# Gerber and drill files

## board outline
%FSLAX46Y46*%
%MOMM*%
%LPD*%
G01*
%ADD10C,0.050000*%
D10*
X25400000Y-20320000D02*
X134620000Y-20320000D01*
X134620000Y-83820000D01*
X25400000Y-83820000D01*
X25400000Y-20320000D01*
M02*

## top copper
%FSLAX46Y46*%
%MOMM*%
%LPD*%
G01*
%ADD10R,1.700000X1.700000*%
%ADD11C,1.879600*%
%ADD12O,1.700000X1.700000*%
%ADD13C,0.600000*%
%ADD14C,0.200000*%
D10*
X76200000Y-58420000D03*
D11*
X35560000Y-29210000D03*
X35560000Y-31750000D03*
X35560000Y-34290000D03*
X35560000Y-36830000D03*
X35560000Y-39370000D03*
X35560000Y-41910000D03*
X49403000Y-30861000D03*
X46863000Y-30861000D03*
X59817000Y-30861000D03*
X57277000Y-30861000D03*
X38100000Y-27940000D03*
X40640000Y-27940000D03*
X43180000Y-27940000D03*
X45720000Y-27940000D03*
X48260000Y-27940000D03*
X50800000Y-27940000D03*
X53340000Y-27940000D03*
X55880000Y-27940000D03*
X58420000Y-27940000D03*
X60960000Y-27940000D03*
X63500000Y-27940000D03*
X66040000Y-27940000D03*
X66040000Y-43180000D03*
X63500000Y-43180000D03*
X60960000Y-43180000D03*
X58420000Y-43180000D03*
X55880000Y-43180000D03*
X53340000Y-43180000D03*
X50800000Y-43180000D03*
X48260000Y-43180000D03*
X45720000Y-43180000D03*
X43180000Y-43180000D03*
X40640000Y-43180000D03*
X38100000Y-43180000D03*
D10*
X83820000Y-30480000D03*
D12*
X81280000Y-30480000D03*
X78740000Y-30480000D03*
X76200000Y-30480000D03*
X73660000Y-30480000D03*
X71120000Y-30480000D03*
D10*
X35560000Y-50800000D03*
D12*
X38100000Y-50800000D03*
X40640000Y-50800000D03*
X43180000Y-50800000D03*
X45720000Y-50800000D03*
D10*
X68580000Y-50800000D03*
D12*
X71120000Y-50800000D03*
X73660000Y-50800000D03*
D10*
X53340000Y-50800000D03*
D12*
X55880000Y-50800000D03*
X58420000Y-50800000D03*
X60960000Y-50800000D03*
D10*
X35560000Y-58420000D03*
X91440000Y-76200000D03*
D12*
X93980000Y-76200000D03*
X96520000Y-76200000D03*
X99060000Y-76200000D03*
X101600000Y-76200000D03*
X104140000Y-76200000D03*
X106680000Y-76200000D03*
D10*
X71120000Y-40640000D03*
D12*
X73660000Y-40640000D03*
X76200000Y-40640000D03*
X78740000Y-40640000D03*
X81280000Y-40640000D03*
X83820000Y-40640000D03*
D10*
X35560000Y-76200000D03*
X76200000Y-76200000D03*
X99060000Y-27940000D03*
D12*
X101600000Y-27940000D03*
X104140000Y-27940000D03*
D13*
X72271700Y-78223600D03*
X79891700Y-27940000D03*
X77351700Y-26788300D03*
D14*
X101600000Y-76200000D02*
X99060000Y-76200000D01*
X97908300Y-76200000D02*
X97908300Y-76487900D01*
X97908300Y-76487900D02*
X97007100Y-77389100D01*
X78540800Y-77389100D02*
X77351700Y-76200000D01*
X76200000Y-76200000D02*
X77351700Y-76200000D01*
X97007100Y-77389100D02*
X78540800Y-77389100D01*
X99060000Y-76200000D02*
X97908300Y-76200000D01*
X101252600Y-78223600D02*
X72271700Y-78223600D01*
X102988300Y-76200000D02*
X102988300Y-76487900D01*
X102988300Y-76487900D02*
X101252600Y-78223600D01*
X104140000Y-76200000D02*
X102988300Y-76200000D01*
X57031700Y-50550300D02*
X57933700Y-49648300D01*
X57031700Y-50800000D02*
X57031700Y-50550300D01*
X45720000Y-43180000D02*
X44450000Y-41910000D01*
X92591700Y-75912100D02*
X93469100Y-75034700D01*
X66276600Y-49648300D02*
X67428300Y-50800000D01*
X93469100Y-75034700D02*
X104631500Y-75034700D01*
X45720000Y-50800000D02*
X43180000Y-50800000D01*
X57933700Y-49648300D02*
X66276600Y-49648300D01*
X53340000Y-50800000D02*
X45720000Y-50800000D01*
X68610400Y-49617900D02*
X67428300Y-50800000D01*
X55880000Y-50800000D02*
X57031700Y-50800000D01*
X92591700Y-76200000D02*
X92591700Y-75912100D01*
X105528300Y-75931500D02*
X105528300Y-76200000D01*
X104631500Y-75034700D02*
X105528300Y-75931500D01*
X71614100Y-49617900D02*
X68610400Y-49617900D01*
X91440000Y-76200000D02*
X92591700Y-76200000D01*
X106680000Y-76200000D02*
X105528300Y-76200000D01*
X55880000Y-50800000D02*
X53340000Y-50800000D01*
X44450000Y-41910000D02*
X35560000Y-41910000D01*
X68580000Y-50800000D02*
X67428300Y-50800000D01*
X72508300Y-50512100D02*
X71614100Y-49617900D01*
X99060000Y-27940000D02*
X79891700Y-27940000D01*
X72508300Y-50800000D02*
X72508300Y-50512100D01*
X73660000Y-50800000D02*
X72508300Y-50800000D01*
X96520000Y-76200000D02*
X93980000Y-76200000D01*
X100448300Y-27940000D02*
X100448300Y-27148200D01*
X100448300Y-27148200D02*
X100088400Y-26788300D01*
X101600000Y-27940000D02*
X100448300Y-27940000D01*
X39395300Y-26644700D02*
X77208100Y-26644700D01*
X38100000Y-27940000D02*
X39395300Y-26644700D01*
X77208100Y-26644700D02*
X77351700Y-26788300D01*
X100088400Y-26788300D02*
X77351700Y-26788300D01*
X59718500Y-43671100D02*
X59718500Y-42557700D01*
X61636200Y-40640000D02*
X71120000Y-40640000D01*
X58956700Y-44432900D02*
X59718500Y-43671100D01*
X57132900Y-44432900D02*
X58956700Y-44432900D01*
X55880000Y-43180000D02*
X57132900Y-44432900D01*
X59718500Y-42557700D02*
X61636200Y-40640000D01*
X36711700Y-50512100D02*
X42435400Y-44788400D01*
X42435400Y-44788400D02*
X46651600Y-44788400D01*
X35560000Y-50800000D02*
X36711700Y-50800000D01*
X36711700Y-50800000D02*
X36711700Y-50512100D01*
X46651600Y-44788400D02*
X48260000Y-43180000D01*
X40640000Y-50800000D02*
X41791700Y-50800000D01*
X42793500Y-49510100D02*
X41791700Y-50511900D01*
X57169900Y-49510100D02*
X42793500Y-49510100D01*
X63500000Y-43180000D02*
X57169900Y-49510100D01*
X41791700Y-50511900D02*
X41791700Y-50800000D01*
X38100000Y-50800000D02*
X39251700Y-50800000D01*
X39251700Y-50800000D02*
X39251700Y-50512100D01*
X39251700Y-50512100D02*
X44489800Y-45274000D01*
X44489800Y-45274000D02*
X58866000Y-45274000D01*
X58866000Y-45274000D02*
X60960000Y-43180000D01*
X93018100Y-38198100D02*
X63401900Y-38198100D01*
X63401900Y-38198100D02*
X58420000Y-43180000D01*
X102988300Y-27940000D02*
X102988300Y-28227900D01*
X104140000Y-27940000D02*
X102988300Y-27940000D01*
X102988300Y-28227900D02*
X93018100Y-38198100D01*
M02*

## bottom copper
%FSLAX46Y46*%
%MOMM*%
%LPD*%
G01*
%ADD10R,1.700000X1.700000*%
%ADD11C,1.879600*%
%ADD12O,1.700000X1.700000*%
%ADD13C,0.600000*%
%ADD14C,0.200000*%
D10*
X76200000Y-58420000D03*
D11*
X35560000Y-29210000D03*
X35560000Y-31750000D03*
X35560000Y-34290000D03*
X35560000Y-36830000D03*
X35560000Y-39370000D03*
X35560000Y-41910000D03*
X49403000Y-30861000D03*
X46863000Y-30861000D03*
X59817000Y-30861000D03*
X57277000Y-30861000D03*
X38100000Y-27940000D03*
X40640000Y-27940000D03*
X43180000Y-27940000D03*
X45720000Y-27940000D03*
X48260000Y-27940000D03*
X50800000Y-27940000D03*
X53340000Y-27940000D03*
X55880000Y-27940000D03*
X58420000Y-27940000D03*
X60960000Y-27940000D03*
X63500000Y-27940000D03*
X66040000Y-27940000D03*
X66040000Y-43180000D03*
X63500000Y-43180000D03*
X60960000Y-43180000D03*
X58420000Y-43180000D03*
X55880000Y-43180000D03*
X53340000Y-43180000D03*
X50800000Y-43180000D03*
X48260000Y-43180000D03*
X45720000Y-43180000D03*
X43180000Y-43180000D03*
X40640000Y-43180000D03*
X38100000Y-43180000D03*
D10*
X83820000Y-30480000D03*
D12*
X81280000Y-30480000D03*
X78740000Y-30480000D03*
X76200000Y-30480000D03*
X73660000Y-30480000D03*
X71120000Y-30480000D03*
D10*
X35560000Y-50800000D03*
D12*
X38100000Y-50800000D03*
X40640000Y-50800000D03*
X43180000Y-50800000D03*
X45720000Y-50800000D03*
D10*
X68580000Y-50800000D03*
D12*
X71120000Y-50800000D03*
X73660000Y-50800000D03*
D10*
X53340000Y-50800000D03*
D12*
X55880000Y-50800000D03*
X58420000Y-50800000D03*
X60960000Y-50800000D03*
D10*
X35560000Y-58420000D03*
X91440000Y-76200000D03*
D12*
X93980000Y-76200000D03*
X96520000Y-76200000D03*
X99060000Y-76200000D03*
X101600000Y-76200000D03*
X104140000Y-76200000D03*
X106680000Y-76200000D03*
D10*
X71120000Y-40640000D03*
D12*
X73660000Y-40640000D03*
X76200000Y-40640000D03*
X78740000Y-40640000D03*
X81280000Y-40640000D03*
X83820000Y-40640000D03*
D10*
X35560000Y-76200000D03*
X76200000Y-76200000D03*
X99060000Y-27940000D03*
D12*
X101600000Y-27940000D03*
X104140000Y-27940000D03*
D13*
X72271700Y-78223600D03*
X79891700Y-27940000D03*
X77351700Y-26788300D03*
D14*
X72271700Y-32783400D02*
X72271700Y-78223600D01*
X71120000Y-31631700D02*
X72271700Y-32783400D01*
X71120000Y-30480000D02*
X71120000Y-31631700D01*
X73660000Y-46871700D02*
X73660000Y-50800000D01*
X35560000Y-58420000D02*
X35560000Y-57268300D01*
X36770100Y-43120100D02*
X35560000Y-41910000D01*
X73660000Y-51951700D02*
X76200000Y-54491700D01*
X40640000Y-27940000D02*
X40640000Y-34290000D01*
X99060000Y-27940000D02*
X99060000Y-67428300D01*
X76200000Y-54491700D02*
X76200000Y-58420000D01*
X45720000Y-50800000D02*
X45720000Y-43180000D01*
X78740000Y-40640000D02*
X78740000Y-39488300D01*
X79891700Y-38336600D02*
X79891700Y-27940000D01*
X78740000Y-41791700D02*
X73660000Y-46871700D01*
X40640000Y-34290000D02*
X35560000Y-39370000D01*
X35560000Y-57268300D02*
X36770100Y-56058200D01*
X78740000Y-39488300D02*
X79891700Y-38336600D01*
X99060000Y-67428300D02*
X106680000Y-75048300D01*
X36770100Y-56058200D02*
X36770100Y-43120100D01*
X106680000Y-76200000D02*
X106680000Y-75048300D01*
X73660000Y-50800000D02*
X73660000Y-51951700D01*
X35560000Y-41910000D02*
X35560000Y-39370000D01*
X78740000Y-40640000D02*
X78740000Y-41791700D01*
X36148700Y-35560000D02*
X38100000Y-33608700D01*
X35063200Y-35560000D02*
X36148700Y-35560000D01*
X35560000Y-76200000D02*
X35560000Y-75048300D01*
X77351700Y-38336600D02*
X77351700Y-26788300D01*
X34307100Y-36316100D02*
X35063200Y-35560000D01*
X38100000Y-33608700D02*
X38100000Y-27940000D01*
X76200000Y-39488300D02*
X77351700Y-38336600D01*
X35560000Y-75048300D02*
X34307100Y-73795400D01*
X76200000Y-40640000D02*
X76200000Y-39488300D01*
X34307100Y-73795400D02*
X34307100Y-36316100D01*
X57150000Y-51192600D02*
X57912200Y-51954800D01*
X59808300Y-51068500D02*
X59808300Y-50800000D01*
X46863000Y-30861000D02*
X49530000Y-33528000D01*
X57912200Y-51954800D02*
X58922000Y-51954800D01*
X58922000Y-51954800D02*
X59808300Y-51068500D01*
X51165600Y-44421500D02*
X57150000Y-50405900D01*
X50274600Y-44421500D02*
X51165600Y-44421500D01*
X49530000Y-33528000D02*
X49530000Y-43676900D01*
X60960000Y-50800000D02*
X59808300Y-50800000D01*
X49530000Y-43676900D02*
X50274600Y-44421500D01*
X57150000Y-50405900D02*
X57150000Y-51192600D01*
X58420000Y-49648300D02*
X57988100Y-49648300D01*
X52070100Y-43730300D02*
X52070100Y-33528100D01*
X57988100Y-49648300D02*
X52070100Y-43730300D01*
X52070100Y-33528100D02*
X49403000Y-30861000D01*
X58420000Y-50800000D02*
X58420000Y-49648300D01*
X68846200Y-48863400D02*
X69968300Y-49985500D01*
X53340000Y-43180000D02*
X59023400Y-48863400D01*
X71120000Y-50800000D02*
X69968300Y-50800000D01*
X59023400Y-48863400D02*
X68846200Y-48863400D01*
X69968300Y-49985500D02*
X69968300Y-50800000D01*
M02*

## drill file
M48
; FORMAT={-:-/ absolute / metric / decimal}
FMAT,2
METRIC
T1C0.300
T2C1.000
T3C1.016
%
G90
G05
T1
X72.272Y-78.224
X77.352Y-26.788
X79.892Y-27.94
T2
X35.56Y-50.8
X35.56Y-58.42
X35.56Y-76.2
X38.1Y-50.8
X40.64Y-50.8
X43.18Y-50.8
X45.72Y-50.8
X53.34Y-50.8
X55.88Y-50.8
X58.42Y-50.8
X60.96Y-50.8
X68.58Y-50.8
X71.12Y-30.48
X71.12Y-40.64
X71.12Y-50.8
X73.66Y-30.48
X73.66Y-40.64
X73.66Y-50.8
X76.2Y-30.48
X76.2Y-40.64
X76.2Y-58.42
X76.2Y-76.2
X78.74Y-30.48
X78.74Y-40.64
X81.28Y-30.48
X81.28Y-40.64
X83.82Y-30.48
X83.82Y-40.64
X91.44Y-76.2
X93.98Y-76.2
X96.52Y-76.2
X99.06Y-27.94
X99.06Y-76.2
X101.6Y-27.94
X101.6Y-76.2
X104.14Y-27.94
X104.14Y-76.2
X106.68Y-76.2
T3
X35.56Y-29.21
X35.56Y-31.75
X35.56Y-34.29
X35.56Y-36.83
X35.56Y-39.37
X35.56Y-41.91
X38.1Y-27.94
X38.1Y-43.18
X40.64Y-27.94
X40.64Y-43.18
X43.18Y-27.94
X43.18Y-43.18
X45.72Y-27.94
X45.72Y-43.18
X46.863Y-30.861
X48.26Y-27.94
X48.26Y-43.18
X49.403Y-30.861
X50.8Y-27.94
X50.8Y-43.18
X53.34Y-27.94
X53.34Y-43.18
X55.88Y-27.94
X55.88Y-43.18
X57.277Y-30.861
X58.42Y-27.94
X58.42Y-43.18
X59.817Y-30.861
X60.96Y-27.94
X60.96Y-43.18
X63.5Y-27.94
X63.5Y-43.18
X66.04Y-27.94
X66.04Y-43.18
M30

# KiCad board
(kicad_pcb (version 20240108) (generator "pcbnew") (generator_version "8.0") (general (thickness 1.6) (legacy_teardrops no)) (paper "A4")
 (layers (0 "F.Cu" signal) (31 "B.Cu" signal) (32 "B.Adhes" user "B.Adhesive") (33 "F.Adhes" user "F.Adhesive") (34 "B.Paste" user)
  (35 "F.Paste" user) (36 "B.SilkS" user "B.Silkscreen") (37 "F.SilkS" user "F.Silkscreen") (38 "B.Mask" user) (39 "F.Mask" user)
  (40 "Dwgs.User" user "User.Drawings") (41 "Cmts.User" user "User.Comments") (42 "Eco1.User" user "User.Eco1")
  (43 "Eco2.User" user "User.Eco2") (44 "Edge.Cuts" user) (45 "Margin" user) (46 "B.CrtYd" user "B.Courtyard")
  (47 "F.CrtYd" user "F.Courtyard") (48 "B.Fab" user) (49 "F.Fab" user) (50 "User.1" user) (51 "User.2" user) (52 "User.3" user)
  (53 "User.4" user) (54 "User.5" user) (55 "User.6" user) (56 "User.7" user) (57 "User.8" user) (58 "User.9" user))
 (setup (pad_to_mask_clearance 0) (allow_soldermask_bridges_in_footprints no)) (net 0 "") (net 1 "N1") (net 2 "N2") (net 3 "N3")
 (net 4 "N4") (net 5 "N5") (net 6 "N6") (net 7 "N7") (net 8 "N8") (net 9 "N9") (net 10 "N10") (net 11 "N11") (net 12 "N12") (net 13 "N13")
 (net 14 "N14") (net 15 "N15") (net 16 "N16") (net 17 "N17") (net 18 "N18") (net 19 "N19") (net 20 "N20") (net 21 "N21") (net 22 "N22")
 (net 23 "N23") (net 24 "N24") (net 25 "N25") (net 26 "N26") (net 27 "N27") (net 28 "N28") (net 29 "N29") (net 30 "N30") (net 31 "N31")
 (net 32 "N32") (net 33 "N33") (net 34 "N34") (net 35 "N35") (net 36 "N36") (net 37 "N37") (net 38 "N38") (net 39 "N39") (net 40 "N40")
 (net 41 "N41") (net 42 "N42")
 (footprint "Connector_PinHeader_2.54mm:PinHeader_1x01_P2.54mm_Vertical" (layer "F.Cu") (at 76.2 58.42)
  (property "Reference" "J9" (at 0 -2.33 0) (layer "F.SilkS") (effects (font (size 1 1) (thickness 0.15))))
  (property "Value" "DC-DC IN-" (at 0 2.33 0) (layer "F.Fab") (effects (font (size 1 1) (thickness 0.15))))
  (pad "1" thru_hole rect (at 0 0) (size 1.7 1.7) (drill 1) (layers "*.Cu" "*.Mask") (remove_unused_layers no) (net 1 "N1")))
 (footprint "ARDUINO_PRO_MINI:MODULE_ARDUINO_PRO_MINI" (layer "F.Cu") (at 50.8 35.56 90)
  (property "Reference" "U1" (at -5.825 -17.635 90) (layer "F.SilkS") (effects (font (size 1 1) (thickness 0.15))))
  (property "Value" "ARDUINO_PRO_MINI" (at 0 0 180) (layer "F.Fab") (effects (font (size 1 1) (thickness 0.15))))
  (pad "JP1_1" thru_hole circle (at 6.35 -15.24 90) (size 1.8796 1.8796) (drill 1.016) (layers "*.Cu" "*.Mask") (remove_unused_layers no)
   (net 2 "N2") (solder_mask_margin 0.102))
  (pad "JP1_2" thru_hole circle (at 3.81 -15.24 90) (size 1.8796 1.8796) (drill 1.016) (layers "*.Cu" "*.Mask") (remove_unused_layers no)
   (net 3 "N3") (solder_mask_margin 0.102))
  (pad "JP1_3" thru_hole circle (at 1.27 -15.24 90) (size 1.8796 1.8796) (drill 1.016) (layers "*.Cu" "*.Mask") (remove_unused_layers no)
   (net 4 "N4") (solder_mask_margin 0.102))
  (pad "JP1_4" thru_hole circle (at -1.27 -15.24 90) (size 1.8796 1.8796) (drill 1.016) (layers "*.Cu" "*.Mask") (remove_unused_layers no)
   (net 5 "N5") (solder_mask_margin 0.102))
  (pad "JP1_5" thru_hole circle (at -3.81 -15.24 90) (size 1.8796 1.8796) (drill 1.016) (layers "*.Cu" "*.Mask") (remove_unused_layers no)
   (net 1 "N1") (solder_mask_margin 0.102))
  (pad "JP1_6" thru_hole circle (at -6.35 -15.24 90) (size 1.8796 1.8796) (drill 1.016) (layers "*.Cu" "*.Mask") (remove_unused_layers no)
   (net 1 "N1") (solder_mask_margin 0.102))
  (pad "JP2_1" thru_hole circle (at 4.699 -1.397 90) (size 1.8796 1.8796) (drill 1.016) (layers "*.Cu" "*.Mask") (remove_unused_layers no)
   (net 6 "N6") (solder_mask_margin 0.102))
  (pad "JP2_2" thru_hole circle (at 4.699 -3.937 90) (size 1.8796 1.8796) (drill 1.016) (layers "*.Cu" "*.Mask") (remove_unused_layers no)
   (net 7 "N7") (solder_mask_margin 0.102))
  (pad "JP3_1" thru_hole circle (at 4.699 9.017 90) (size 1.8796 1.8796) (drill 1.016) (layers "*.Cu" "*.Mask") (remove_unused_layers no)
   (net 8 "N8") (solder_mask_margin 0.102))
  (pad "JP3_2" thru_hole circle (at 4.699 6.477 90) (size 1.8796 1.8796) (drill 1.016) (layers "*.Cu" "*.Mask") (remove_unused_layers no)
   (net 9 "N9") (solder_mask_margin 0.102))
  (pad "JP6_1" thru_hole circle (at 7.62 -12.7 90) (size 1.8796 1.8796) (drill 1.016) (layers "*.Cu" "*.Mask") (remove_unused_layers no)
   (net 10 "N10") (solder_mask_margin 0.102))
  (pad "JP6_2" thru_hole circle (at 7.62 -10.16 90) (size 1.8796 1.8796) (drill 1.016) (layers "*.Cu" "*.Mask") (remove_unused_layers no)
   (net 1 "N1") (solder_mask_margin 0.102))
  (pad "JP6_3" thru_hole circle (at 7.62 -7.62 90) (size 1.8796 1.8796) (drill 1.016) (layers "*.Cu" "*.Mask") (remove_unused_layers no)
   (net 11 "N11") (solder_mask_margin 0.102))
  (pad "JP6_4" thru_hole circle (at 7.62 -5.08 90) (size 1.8796 1.8796) (drill 1.016) (layers "*.Cu" "*.Mask") (remove_unused_layers no)
   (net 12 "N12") (solder_mask_margin 0.102))
  (pad "JP6_5" thru_hole circle (at 7.62 -2.54 90) (size 1.8796 1.8796) (drill 1.016) (layers "*.Cu" "*.Mask") (remove_unused_layers no)
   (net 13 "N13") (solder_mask_margin 0.102))
  (pad "JP6_6" thru_hole circle (at 7.62 0 90) (size 1.8796 1.8796) (drill 1.016) (layers "*.Cu" "*.Mask") (remove_unused_layers no)
   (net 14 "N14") (solder_mask_margin 0.102))
  (pad "JP6_7" thru_hole circle (at 7.62 2.54 90) (size 1.8796 1.8796) (drill 1.016) (layers "*.Cu" "*.Mask") (remove_unused_layers no)
   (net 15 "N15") (solder_mask_margin 0.102))
  (pad "JP6_8" thru_hole circle (at 7.62 5.08 90) (size 1.8796 1.8796) (drill 1.016) (layers "*.Cu" "*.Mask") (remove_unused_layers no)
   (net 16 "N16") (solder_mask_margin 0.102))
  (pad "JP6_9" thru_hole circle (at 7.62 7.62 90) (size 1.8796 1.8796) (drill 1.016) (layers "*.Cu" "*.Mask") (remove_unused_layers no)
   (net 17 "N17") (solder_mask_margin 0.102))
  (pad "JP6_10" thru_hole circle (at 7.62 10.16 90) (size 1.8796 1.8796) (drill 1.016) (layers "*.Cu" "*.Mask") (remove_unused_layers no)
   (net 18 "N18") (solder_mask_margin 0.102))
  (pad "JP6_11" thru_hole circle (at 7.62 12.7 90) (size 1.8796 1.8796) (drill 1.016) (layers "*.Cu" "*.Mask") (remove_unused_layers no)
   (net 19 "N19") (solder_mask_margin 0.102))
  (pad "JP6_12" thru_hole circle (at 7.62 15.24 90) (size 1.8796 1.8796) (drill 1.016) (layers "*.Cu" "*.Mask") (remove_unused_layers no)
   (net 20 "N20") (solder_mask_margin 0.102))
  (pad "JP7_1" thru_hole circle (at -7.62 15.24 90) (size 1.8796 1.8796) (drill 1.016) (layers "*.Cu" "*.Mask") (remove_unused_layers no)
   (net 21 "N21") (solder_mask_margin 0.102))
  (pad "JP7_2" thru_hole circle (at -7.62 12.7 90) (size 1.8796 1.8796) (drill 1.016) (layers "*.Cu" "*.Mask") (remove_unused_layers no)
   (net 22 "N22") (solder_mask_margin 0.102))
  (pad "JP7_3" thru_hole circle (at -7.62 10.16 90) (size 1.8796 1.8796) (drill 1.016) (layers "*.Cu" "*.Mask") (remove_unused_layers no)
   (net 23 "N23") (solder_mask_margin 0.102))
  (pad "JP7_4" thru_hole circle (at -7.62 7.62 90) (size 1.8796 1.8796) (drill 1.016) (layers "*.Cu" "*.Mask") (remove_unused_layers no)
   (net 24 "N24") (solder_mask_margin 0.102))
  (pad "JP7_5" thru_hole circle (at -7.62 5.08 90) (size 1.8796 1.8796) (drill 1.016) (layers "*.Cu" "*.Mask") (remove_unused_layers no)
   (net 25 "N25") (solder_mask_margin 0.102))
  (pad "JP7_6" thru_hole circle (at -7.62 2.54 90) (size 1.8796 1.8796) (drill 1.016) (layers "*.Cu" "*.Mask") (remove_unused_layers no)
   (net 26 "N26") (solder_mask_margin 0.102))
  (pad "JP7_7" thru_hole circle (at -7.62 0 90) (size 1.8796 1.8796) (drill 1.016) (layers "*.Cu" "*.Mask") (remove_unused_layers no)
   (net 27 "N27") (solder_mask_margin 0.102))
  (pad "JP7_8" thru_hole circle (at -7.62 -2.54 90) (size 1.8796 1.8796) (drill 1.016) (layers "*.Cu" "*.Mask") (remove_unused_layers no)
   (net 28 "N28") (solder_mask_margin 0.102))
  (pad "JP7_9" thru_hole circle (at -7.62 -5.08 90) (size 1.8796 1.8796) (drill 1.016) (layers "*.Cu" "*.Mask") (remove_unused_layers no)
   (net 1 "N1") (solder_mask_margin 0.102))
  (pad "JP7_10" thru_hole circle (at -7.62 -7.62 90) (size 1.8796 1.8796) (drill 1.016) (layers "*.Cu" "*.Mask") (remove_unused_layers no)
   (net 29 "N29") (solder_mask_margin 0.102))
  (pad "JP7_11" thru_hole circle (at -7.62 -10.16 90) (size 1.8796 1.8796) (drill 1.016) (layers "*.Cu" "*.Mask") (remove_unused_layers no)
   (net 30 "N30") (solder_mask_margin 0.102))
  (pad "JP7_12" thru_hole circle (at -7.62 -12.7 90) (size 1.8796 1.8796) (drill 1.016) (layers "*.Cu" "*.Mask") (remove_unused_layers no)
   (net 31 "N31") (solder_mask_margin 0.102)))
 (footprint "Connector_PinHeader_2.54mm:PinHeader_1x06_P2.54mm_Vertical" (layer "F.Cu") (at 83.82 30.48 -90)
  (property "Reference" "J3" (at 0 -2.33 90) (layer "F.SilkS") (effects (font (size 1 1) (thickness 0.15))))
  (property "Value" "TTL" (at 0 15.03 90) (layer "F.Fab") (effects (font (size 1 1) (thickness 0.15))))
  (pad "1" thru_hole rect (at 0 0 270) (size 1.7 1.7) (drill 1) (layers "*.Cu" "*.Mask") (remove_unused_layers no) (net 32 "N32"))
  (pad "2" thru_hole oval (at 0 2.54 270) (size 1.7 1.7) (drill 1) (layers "*.Cu" "*.Mask") (remove_unused_layers no) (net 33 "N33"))
  (pad "3" thru_hole oval (at 0 5.08 270) (size 1.7 1.7) (drill 1) (layers "*.Cu" "*.Mask") (remove_unused_layers no) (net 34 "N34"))
  (pad "4" thru_hole oval (at 0 7.62 270) (size 1.7 1.7) (drill 1) (layers "*.Cu" "*.Mask") (remove_unused_layers no) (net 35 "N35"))
  (pad "5" thru_hole oval (at 0 10.16 270) (size 1.7 1.7) (drill 1) (layers "*.Cu" "*.Mask") (remove_unused_layers no) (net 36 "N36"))
  (pad "6" thru_hole oval (at 0 12.7 270) (size 1.7 1.7) (drill 1) (layers "*.Cu" "*.Mask") (remove_unused_layers no) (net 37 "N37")))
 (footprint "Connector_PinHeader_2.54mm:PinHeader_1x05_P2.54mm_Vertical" (layer "F.Cu") (at 35.56 50.8 90)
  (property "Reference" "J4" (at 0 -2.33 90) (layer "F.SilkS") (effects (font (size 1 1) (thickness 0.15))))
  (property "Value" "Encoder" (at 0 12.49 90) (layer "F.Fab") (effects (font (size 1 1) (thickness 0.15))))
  (pad "1" thru_hole rect (at 0 0 90) (size 1.7 1.7) (drill 1) (layers "*.Cu" "*.Mask") (remove_unused_layers no) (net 28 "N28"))
  (pad "2" thru_hole oval (at 0 2.54 90) (size 1.7 1.7) (drill 1) (layers "*.Cu" "*.Mask") (remove_unused_layers no) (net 23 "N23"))
  (pad "3" thru_hole oval (at 0 5.08 90) (size 1.7 1.7) (drill 1) (layers "*.Cu" "*.Mask") (remove_unused_layers no) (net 22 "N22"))
  (pad "4" thru_hole oval (at 0 7.62 90) (size 1.7 1.7) (drill 1) (layers "*.Cu" "*.Mask") (remove_unused_layers no) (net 1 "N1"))
  (pad "5" thru_hole oval (at 0 10.16 90) (size 1.7 1.7) (drill 1) (layers "*.Cu" "*.Mask") (remove_unused_layers no) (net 1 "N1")))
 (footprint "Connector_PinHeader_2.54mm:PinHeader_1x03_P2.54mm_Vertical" (layer "F.Cu") (at 68.58 50.8 90)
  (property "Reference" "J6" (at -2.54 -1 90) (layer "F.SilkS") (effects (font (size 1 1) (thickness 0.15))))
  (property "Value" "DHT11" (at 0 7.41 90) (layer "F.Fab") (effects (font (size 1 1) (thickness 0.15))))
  (pad "1" thru_hole rect (at 0 0 90) (size 1.7 1.7) (drill 1) (layers "*.Cu" "*.Mask") (remove_unused_layers no) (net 1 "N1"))
  (pad "2" thru_hole oval (at 0 2.54 90) (size 1.7 1.7) (drill 1) (layers "*.Cu" "*.Mask") (remove_unused_layers no) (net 26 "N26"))
  (pad "3" thru_hole oval (at 0 5.08 90) (size 1.7 1.7) (drill 1) (layers "*.Cu" "*.Mask") (remove_unused_layers no) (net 1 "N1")))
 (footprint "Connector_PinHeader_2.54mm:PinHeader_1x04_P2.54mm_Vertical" (layer "F.Cu") (at 53.34 50.8 90)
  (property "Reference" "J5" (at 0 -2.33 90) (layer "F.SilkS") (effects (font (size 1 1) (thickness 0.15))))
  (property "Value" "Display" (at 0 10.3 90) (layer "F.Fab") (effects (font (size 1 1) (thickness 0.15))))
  (pad "1" thru_hole rect (at 0 0 90) (size 1.7 1.7) (drill 1) (layers "*.Cu" "*.Mask") (remove_unused_layers no) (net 1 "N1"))
  (pad "2" thru_hole oval (at 0 2.54 90) (size 1.7 1.7) (drill 1) (layers "*.Cu" "*.Mask") (remove_unused_layers no) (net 1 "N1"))
  (pad "3" thru_hole oval (at 0 5.08 90) (size 1.7 1.7) (drill 1) (layers "*.Cu" "*.Mask") (remove_unused_layers no) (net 6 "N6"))
  (pad "4" thru_hole oval (at 0 7.62 90) (size 1.7 1.7) (drill 1) (layers "*.Cu" "*.Mask") (remove_unused_layers no) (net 7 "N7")))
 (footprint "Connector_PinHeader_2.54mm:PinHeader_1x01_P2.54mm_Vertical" (layer "F.Cu") (at 35.56 58.42)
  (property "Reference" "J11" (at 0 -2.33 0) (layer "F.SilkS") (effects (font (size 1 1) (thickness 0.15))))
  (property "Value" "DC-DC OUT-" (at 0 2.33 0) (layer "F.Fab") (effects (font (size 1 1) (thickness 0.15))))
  (pad "1" thru_hole rect (at 0 0) (size 1.7 1.7) (drill 1) (layers "*.Cu" "*.Mask") (remove_unused_layers no) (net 1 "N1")))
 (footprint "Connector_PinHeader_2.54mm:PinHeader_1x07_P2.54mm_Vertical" (layer "F.Cu") (at 91.44 76.2 90)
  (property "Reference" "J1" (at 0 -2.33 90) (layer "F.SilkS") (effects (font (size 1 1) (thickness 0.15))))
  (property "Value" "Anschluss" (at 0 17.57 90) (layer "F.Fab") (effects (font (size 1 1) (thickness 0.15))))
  (pad "1" thru_hole rect (at 0 0 90) (size 1.7 1.7) (drill 1) (layers "*.Cu" "*.Mask") (remove_unused_layers no) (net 1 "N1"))
  (pad "2" thru_hole oval (at 0 2.54 90) (size 1.7 1.7) (drill 1) (layers "*.Cu" "*.Mask") (remove_unused_layers no) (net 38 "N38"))
  (pad "3" thru_hole oval (at 0 5.08 90) (size 1.7 1.7) (drill 1) (layers "*.Cu" "*.Mask") (remove_unused_layers no) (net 38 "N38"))
  (pad "4" thru_hole oval (at 0 7.62 90) (size 1.7 1.7) (drill 1) (layers "*.Cu" "*.Mask") (remove_unused_layers no) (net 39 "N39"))
  (pad "5" thru_hole oval (at 0 10.16 90) (size 1.7 1.7) (drill 1) (layers "*.Cu" "*.Mask") (remove_unused_layers no) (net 39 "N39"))
  (pad "6" thru_hole oval (at 0 12.7 90) (size 1.7 1.7) (drill 1) (layers "*.Cu" "*.Mask") (remove_unused_layers no) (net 37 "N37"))
  (pad "7" thru_hole oval (at 0 15.24 90) (size 1.7 1.7) (drill 1) (layers "*.Cu" "*.Mask") (remove_unused_layers no) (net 1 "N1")))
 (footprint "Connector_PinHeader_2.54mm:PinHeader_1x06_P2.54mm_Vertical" (layer "F.Cu") (at 71.12 40.64 90)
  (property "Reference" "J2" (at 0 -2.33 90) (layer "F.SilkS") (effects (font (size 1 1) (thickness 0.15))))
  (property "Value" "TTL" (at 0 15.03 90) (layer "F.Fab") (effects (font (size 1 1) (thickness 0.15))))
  (pad "1" thru_hole rect (at 0 0 90) (size 1.7 1.7) (drill 1) (layers "*.Cu" "*.Mask") (remove_unused_layers no) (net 25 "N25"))
  (pad "2" thru_hole oval (at 0 2.54 90) (size 1.7 1.7) (drill 1) (layers "*.Cu" "*.Mask") (remove_unused_layers no) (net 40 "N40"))
  (pad "3" thru_hole oval (at 0 5.08 90) (size 1.7 1.7) (drill 1) (layers "*.Cu" "*.Mask") (remove_unused_layers no) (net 10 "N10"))
  (pad "4" thru_hole oval (at 0 7.62 90) (size 1.7 1.7) (drill 1) (layers "*.Cu" "*.Mask") (remove_unused_layers no) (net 1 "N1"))
  (pad "5" thru_hole oval (at 0 10.16 90) (size 1.7 1.7) (drill 1) (layers "*.Cu" "*.Mask") (remove_unused_layers no) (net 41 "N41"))
  (pad "6" thru_hole oval (at 0 12.7 90) (size 1.7 1.7) (drill 1) (layers "*.Cu" "*.Mask") (remove_unused_layers no) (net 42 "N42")))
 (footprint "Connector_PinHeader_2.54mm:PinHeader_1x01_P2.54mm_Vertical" (layer "F.Cu") (at 35.56 76.2)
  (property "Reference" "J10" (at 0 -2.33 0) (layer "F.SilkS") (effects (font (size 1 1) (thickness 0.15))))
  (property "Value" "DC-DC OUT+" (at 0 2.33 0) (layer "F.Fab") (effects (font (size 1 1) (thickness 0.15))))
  (pad "1" thru_hole rect (at 0 0) (size 1.7 1.7) (drill 1) (layers "*.Cu" "*.Mask") (remove_unused_layers no) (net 10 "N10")))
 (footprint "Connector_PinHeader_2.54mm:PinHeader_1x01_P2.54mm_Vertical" (layer "F.Cu") (at 76.2 76.2)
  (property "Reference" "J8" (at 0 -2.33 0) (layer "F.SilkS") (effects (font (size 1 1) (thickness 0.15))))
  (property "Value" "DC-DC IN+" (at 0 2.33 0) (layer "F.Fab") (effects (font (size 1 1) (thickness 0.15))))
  (pad "1" thru_hole rect (at 0 0) (size 1.7 1.7) (drill 1) (layers "*.Cu" "*.Mask") (remove_unused_layers no) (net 39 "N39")))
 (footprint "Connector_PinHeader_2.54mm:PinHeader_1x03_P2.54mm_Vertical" (layer "F.Cu") (at 99.06 27.94 90)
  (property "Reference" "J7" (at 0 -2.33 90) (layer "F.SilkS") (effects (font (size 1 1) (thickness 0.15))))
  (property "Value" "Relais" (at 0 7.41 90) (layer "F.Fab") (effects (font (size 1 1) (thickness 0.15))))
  (pad "1" thru_hole rect (at 0 0 90) (size 1.7 1.7) (drill 1) (layers "*.Cu" "*.Mask") (remove_unused_layers no) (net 1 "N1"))
  (pad "2" thru_hole oval (at 0 2.54 90) (size 1.7 1.7) (drill 1) (layers "*.Cu" "*.Mask") (remove_unused_layers no) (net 10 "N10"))
  (pad "3" thru_hole oval (at 0 5.08 90) (size 1.7 1.7) (drill 1) (layers "*.Cu" "*.Mask") (remove_unused_layers no) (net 24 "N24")))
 (gr_rect (start 25.4 20.32) (end 134.62 83.82) (stroke (width 0.05) (type default)) (fill none) (layer "Edge.Cuts"))
 (segment (start 101.6 76.2) (end 99.06 76.2) (width 0.2) (layer "F.Cu") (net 39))
 (segment (start 97.9083 76.2) (end 97.9083 76.4879) (width 0.2) (layer "F.Cu") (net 39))
 (segment (start 97.9083 76.4879) (end 97.0071 77.3891) (width 0.2) (layer "F.Cu") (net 39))
 (segment (start 78.5408 77.3891) (end 77.3517 76.2) (width 0.2) (layer "F.Cu") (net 39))
 (segment (start 76.2 76.2) (end 77.3517 76.2) (width 0.2) (layer "F.Cu") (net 39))
 (segment (start 97.0071 77.3891) (end 78.5408 77.3891) (width 0.2) (layer "F.Cu") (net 39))
 (segment (start 99.06 76.2) (end 97.9083 76.2) (width 0.2) (layer "F.Cu") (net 39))
 (segment (start 101.2526 78.2236) (end 72.2717 78.2236) (width 0.2) (layer "F.Cu") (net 37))
 (segment (start 102.9883 76.2) (end 102.9883 76.4879) (width 0.2) (layer "F.Cu") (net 37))
 (segment (start 102.9883 76.4879) (end 101.2526 78.2236) (width 0.2) (layer "F.Cu") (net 37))
 (segment (start 104.14 76.2) (end 102.9883 76.2) (width 0.2) (layer "F.Cu") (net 37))
 (via (at 72.2717 78.2236) (size 0.6) (drill 0.3) (layers "F.Cu" "B.Cu") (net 37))
 (segment (start 72.2717 32.7834) (end 72.2717 78.2236) (width 0.2) (layer "B.Cu") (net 37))
 (segment (start 71.12 31.6317) (end 72.2717 32.7834) (width 0.2) (layer "B.Cu") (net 37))
 (segment (start 71.12 30.48) (end 71.12 31.6317) (width 0.2) (layer "B.Cu") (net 37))
 (segment (start 57.0317 50.5503) (end 57.9337 49.6483) (width 0.2) (layer "F.Cu") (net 1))
 (segment (start 57.0317 50.8) (end 57.0317 50.5503) (width 0.2) (layer "F.Cu") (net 1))
 (segment (start 45.72 43.18) (end 44.45 41.91) (width 0.2) (layer "F.Cu") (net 1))
 (segment (start 92.5917 75.9121) (end 93.4691 75.0347) (width 0.2) (layer "F.Cu") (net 1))
 (segment (start 66.2766 49.6483) (end 67.4283 50.8) (width 0.2) (layer "F.Cu") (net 1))
 (segment (start 93.4691 75.0347) (end 104.6315 75.0347) (width 0.2) (layer "F.Cu") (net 1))
 (segment (start 45.72 50.8) (end 43.18 50.8) (width 0.2) (layer "F.Cu") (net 1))
 (segment (start 57.9337 49.6483) (end 66.2766 49.6483) (width 0.2) (layer "F.Cu") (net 1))
 (segment (start 53.34 50.8) (end 45.72 50.8) (width 0.2) (layer "F.Cu") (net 1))
 (segment (start 68.6104 49.6179) (end 67.4283 50.8) (width 0.2) (layer "F.Cu") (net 1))
 (segment (start 55.88 50.8) (end 57.0317 50.8) (width 0.2) (layer "F.Cu") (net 1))
 (segment (start 92.5917 76.2) (end 92.5917 75.9121) (width 0.2) (layer "F.Cu") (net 1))
 (segment (start 105.5283 75.9315) (end 105.5283 76.2) (width 0.2) (layer "F.Cu") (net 1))
 (segment (start 104.6315 75.0347) (end 105.5283 75.9315) (width 0.2) (layer "F.Cu") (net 1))
 (segment (start 71.6141 49.6179) (end 68.6104 49.6179) (width 0.2) (layer "F.Cu") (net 1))
 (segment (start 91.44 76.2) (end 92.5917 76.2) (width 0.2) (layer "F.Cu") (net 1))
 (segment (start 106.68 76.2) (end 105.5283 76.2) (width 0.2) (layer "F.Cu") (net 1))
 (segment (start 55.88 50.8) (end 53.34 50.8) (width 0.2) (layer "F.Cu") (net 1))
 (segment (start 44.45 41.91) (end 35.56 41.91) (width 0.2) (layer "F.Cu") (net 1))
 (segment (start 68.58 50.8) (end 67.4283 50.8) (width 0.2) (layer "F.Cu") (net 1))
 (segment (start 72.5083 50.5121) (end 71.6141 49.6179) (width 0.2) (layer "F.Cu") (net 1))
 (segment (start 99.06 27.94) (end 79.8917 27.94) (width 0.2) (layer "F.Cu") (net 1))
 (segment (start 72.5083 50.8) (end 72.5083 50.5121) (width 0.2) (layer "F.Cu") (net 1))
 (segment (start 73.66 50.8) (end 72.5083 50.8) (width 0.2) (layer "F.Cu") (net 1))
 (via (at 79.8917 27.94) (size 0.6) (drill 0.3) (layers "F.Cu" "B.Cu") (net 1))
 (segment (start 73.66 46.8717) (end 73.66 50.8) (width 0.2) (layer "B.Cu") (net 1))
 (segment (start 35.56 58.42) (end 35.56 57.2683) (width 0.2) (layer "B.Cu") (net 1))
 (segment (start 36.7701 43.1201) (end 35.56 41.91) (width 0.2) (layer "B.Cu") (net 1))
 (segment (start 73.66 51.9517) (end 76.2 54.4917) (width 0.2) (layer "B.Cu") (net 1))
 (segment (start 40.64 27.94) (end 40.64 34.29) (width 0.2) (layer "B.Cu") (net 1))
 (segment (start 99.06 27.94) (end 99.06 67.4283) (width 0.2) (layer "B.Cu") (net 1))
 (segment (start 76.2 54.4917) (end 76.2 58.42) (width 0.2) (layer "B.Cu") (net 1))
 (segment (start 45.72 50.8) (end 45.72 43.18) (width 0.2) (layer "B.Cu") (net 1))
 (segment (start 78.74 40.64) (end 78.74 39.4883) (width 0.2) (layer "B.Cu") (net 1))
 (segment (start 79.8917 38.3366) (end 79.8917 27.94) (width 0.2) (layer "B.Cu") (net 1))
 (segment (start 78.74 41.7917) (end 73.66 46.8717) (width 0.2) (layer "B.Cu") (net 1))
 (segment (start 40.64 34.29) (end 35.56 39.37) (width 0.2) (layer "B.Cu") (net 1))
 (segment (start 35.56 57.2683) (end 36.7701 56.0582) (width 0.2) (layer "B.Cu") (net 1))
 (segment (start 78.74 39.4883) (end 79.8917 38.3366) (width 0.2) (layer "B.Cu") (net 1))
 (segment (start 99.06 67.4283) (end 106.68 75.0483) (width 0.2) (layer "B.Cu") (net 1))
 (segment (start 36.7701 56.0582) (end 36.7701 43.1201) (width 0.2) (layer "B.Cu") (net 1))
 (segment (start 106.68 76.2) (end 106.68 75.0483) (width 0.2) (layer "B.Cu") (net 1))
 (segment (start 73.66 50.8) (end 73.66 51.9517) (width 0.2) (layer "B.Cu") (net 1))
 (segment (start 35.56 41.91) (end 35.56 39.37) (width 0.2) (layer "B.Cu") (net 1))
 (segment (start 78.74 40.64) (end 78.74 41.7917) (width 0.2) (layer "B.Cu") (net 1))
 (segment (start 96.52 76.2) (end 93.98 76.2) (width 0.2) (layer "F.Cu") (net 38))
 (segment (start 100.4483 27.94) (end 100.4483 27.1482) (width 0.2) (layer "F.Cu") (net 10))
 (segment (start 100.4483 27.1482) (end 100.0884 26.7883) (width 0.2) (layer "F.Cu") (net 10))
 (segment (start 101.6 27.94) (end 100.4483 27.94) (width 0.2) (layer "F.Cu") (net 10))
 (segment (start 39.3953 26.6447) (end 77.2081 26.6447) (width 0.2) (layer "F.Cu") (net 10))
 (segment (start 38.1 27.94) (end 39.3953 26.6447) (width 0.2) (layer "F.Cu") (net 10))
 (segment (start 77.2081 26.6447) (end 77.3517 26.7883) (width 0.2) (layer "F.Cu") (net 10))
 (segment (start 100.0884 26.7883) (end 77.3517 26.7883) (width 0.2) (layer "F.Cu") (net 10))
 (via (at 77.3517 26.7883) (size 0.6) (drill 0.3) (layers "F.Cu" "B.Cu") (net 10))
 (segment (start 36.1487 35.56) (end 38.1 33.6087) (width 0.2) (layer "B.Cu") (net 10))
 (segment (start 35.0632 35.56) (end 36.1487 35.56) (width 0.2) (layer "B.Cu") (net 10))
 (segment (start 35.56 76.2) (end 35.56 75.0483) (width 0.2) (layer "B.Cu") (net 10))
 (segment (start 77.3517 38.3366) (end 77.3517 26.7883) (width 0.2) (layer "B.Cu") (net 10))
 (segment (start 34.3071 36.3161) (end 35.0632 35.56) (width 0.2) (layer "B.Cu") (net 10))
 (segment (start 38.1 33.6087) (end 38.1 27.94) (width 0.2) (layer "B.Cu") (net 10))
 (segment (start 76.2 39.4883) (end 77.3517 38.3366) (width 0.2) (layer "B.Cu") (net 10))
 (segment (start 35.56 75.0483) (end 34.3071 73.7954) (width 0.2) (layer "B.Cu") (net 10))
 (segment (start 76.2 40.64) (end 76.2 39.4883) (width 0.2) (layer "B.Cu") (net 10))
 (segment (start 34.3071 73.7954) (end 34.3071 36.3161) (width 0.2) (layer "B.Cu") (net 10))
 (segment (start 59.7185 43.6711) (end 59.7185 42.5577) (width 0.2) (layer "F.Cu") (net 25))
 (segment (start 61.6362 40.64) (end 71.12 40.64) (width 0.2) (layer "F.Cu") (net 25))
 (segment (start 58.9567 44.4329) (end 59.7185 43.6711) (width 0.2) (layer "F.Cu") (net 25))
 (segment (start 57.1329 44.4329) (end 58.9567 44.4329) (width 0.2) (layer "F.Cu") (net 25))
 (segment (start 55.88 43.18) (end 57.1329 44.4329) (width 0.2) (layer "F.Cu") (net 25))
 (segment (start 59.7185 42.5577) (end 61.6362 40.64) (width 0.2) (layer "F.Cu") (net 25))
 (segment (start 36.7117 50.5121) (end 42.4354 44.7884) (width 0.2) (layer "F.Cu") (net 28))
 (segment (start 42.4354 44.7884) (end 46.6516 44.7884) (width 0.2) (layer "F.Cu") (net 28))
 (segment (start 35.56 50.8) (end 36.7117 50.8) (width 0.2) (layer "F.Cu") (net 28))
 (segment (start 36.7117 50.8) (end 36.7117 50.5121) (width 0.2) (layer "F.Cu") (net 28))
 (segment (start 46.6516 44.7884) (end 48.26 43.18) (width 0.2) (layer "F.Cu") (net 28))
 (segment (start 40.64 50.8) (end 41.7917 50.8) (width 0.2) (layer "F.Cu") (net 22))
 (segment (start 42.7935 49.5101) (end 41.7917 50.5119) (width 0.2) (layer "F.Cu") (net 22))
 (segment (start 57.1699 49.5101) (end 42.7935 49.5101) (width 0.2) (layer "F.Cu") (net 22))
 (segment (start 63.5 43.18) (end 57.1699 49.5101) (width 0.2) (layer "F.Cu") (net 22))
 (segment (start 41.7917 50.5119) (end 41.7917 50.8) (width 0.2) (layer "F.Cu") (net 22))
 (segment (start 38.1 50.8) (end 39.2517 50.8) (width 0.2) (layer "F.Cu") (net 23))
 (segment (start 39.2517 50.8) (end 39.2517 50.5121) (width 0.2) (layer "F.Cu") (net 23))
 (segment (start 39.2517 50.5121) (end 44.4898 45.274) (width 0.2) (layer "F.Cu") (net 23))
 (segment (start 44.4898 45.274) (end 58.866 45.274) (width 0.2) (layer "F.Cu") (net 23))
 (segment (start 58.866 45.274) (end 60.96 43.18) (width 0.2) (layer "F.Cu") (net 23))
 (segment (start 57.15 51.1926) (end 57.9122 51.9548) (width 0.2) (layer "B.Cu") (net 7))
 (segment (start 59.8083 51.0685) (end 59.8083 50.8) (width 0.2) (layer "B.Cu") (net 7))
 (segment (start 46.863 30.861) (end 49.53 33.528) (width 0.2) (layer "B.Cu") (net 7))
 (segment (start 57.9122 51.9548) (end 58.922 51.9548) (width 0.2) (layer "B.Cu") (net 7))
 (segment (start 58.922 51.9548) (end 59.8083 51.0685) (width 0.2) (layer "B.Cu") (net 7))
 (segment (start 51.1656 44.4215) (end 57.15 50.4059) (width 0.2) (layer "B.Cu") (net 7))
 (segment (start 50.2746 44.4215) (end 51.1656 44.4215) (width 0.2) (layer "B.Cu") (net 7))
 (segment (start 49.53 33.528) (end 49.53 43.6769) (width 0.2) (layer "B.Cu") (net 7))
 (segment (start 60.96 50.8) (end 59.8083 50.8) (width 0.2) (layer "B.Cu") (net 7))
 (segment (start 49.53 43.6769) (end 50.2746 44.4215) (width 0.2) (layer "B.Cu") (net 7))
 (segment (start 57.15 50.4059) (end 57.15 51.1926) (width 0.2) (layer "B.Cu") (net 7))
 (segment (start 58.42 49.6483) (end 57.9881 49.6483) (width 0.2) (layer "B.Cu") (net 6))
 (segment (start 52.0701 43.7303) (end 52.0701 33.5281) (width 0.2) (layer "B.Cu") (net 6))
 (segment (start 57.9881 49.6483) (end 52.0701 43.7303) (width 0.2) (layer "B.Cu") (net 6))
 (segment (start 52.0701 33.5281) (end 49.403 30.861) (width 0.2) (layer "B.Cu") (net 6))
 (segment (start 58.42 50.8) (end 58.42 49.6483) (width 0.2) (layer "B.Cu") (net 6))
 (segment (start 68.8462 48.8634) (end 69.9683 49.9855) (width 0.2) (layer "B.Cu") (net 26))
 (segment (start 53.34 43.18) (end 59.0234 48.8634) (width 0.2) (layer "B.Cu") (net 26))
 (segment (start 71.12 50.8) (end 69.9683 50.8) (width 0.2) (layer "B.Cu") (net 26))
 (segment (start 59.0234 48.8634) (end 68.8462 48.8634) (width 0.2) (layer "B.Cu") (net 26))
 (segment (start 69.9683 49.9855) (end 69.9683 50.8) (width 0.2) (layer "B.Cu") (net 26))
 (segment (start 93.0181 38.1981) (end 63.4019 38.1981) (width 0.2) (layer "F.Cu") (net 24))
 (segment (start 63.4019 38.1981) (end 58.42 43.18) (width 0.2) (layer "F.Cu") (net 24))
 (segment (start 102.9883 27.94) (end 102.9883 28.2279) (width 0.2) (layer "F.Cu") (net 24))
 (segment (start 104.14 27.94) (end 102.9883 27.94) (width 0.2) (layer "F.Cu") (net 24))
 (segment (start 102.9883 28.2279) (end 93.0181 38.1981) (width 0.2) (layer "F.Cu") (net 24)))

